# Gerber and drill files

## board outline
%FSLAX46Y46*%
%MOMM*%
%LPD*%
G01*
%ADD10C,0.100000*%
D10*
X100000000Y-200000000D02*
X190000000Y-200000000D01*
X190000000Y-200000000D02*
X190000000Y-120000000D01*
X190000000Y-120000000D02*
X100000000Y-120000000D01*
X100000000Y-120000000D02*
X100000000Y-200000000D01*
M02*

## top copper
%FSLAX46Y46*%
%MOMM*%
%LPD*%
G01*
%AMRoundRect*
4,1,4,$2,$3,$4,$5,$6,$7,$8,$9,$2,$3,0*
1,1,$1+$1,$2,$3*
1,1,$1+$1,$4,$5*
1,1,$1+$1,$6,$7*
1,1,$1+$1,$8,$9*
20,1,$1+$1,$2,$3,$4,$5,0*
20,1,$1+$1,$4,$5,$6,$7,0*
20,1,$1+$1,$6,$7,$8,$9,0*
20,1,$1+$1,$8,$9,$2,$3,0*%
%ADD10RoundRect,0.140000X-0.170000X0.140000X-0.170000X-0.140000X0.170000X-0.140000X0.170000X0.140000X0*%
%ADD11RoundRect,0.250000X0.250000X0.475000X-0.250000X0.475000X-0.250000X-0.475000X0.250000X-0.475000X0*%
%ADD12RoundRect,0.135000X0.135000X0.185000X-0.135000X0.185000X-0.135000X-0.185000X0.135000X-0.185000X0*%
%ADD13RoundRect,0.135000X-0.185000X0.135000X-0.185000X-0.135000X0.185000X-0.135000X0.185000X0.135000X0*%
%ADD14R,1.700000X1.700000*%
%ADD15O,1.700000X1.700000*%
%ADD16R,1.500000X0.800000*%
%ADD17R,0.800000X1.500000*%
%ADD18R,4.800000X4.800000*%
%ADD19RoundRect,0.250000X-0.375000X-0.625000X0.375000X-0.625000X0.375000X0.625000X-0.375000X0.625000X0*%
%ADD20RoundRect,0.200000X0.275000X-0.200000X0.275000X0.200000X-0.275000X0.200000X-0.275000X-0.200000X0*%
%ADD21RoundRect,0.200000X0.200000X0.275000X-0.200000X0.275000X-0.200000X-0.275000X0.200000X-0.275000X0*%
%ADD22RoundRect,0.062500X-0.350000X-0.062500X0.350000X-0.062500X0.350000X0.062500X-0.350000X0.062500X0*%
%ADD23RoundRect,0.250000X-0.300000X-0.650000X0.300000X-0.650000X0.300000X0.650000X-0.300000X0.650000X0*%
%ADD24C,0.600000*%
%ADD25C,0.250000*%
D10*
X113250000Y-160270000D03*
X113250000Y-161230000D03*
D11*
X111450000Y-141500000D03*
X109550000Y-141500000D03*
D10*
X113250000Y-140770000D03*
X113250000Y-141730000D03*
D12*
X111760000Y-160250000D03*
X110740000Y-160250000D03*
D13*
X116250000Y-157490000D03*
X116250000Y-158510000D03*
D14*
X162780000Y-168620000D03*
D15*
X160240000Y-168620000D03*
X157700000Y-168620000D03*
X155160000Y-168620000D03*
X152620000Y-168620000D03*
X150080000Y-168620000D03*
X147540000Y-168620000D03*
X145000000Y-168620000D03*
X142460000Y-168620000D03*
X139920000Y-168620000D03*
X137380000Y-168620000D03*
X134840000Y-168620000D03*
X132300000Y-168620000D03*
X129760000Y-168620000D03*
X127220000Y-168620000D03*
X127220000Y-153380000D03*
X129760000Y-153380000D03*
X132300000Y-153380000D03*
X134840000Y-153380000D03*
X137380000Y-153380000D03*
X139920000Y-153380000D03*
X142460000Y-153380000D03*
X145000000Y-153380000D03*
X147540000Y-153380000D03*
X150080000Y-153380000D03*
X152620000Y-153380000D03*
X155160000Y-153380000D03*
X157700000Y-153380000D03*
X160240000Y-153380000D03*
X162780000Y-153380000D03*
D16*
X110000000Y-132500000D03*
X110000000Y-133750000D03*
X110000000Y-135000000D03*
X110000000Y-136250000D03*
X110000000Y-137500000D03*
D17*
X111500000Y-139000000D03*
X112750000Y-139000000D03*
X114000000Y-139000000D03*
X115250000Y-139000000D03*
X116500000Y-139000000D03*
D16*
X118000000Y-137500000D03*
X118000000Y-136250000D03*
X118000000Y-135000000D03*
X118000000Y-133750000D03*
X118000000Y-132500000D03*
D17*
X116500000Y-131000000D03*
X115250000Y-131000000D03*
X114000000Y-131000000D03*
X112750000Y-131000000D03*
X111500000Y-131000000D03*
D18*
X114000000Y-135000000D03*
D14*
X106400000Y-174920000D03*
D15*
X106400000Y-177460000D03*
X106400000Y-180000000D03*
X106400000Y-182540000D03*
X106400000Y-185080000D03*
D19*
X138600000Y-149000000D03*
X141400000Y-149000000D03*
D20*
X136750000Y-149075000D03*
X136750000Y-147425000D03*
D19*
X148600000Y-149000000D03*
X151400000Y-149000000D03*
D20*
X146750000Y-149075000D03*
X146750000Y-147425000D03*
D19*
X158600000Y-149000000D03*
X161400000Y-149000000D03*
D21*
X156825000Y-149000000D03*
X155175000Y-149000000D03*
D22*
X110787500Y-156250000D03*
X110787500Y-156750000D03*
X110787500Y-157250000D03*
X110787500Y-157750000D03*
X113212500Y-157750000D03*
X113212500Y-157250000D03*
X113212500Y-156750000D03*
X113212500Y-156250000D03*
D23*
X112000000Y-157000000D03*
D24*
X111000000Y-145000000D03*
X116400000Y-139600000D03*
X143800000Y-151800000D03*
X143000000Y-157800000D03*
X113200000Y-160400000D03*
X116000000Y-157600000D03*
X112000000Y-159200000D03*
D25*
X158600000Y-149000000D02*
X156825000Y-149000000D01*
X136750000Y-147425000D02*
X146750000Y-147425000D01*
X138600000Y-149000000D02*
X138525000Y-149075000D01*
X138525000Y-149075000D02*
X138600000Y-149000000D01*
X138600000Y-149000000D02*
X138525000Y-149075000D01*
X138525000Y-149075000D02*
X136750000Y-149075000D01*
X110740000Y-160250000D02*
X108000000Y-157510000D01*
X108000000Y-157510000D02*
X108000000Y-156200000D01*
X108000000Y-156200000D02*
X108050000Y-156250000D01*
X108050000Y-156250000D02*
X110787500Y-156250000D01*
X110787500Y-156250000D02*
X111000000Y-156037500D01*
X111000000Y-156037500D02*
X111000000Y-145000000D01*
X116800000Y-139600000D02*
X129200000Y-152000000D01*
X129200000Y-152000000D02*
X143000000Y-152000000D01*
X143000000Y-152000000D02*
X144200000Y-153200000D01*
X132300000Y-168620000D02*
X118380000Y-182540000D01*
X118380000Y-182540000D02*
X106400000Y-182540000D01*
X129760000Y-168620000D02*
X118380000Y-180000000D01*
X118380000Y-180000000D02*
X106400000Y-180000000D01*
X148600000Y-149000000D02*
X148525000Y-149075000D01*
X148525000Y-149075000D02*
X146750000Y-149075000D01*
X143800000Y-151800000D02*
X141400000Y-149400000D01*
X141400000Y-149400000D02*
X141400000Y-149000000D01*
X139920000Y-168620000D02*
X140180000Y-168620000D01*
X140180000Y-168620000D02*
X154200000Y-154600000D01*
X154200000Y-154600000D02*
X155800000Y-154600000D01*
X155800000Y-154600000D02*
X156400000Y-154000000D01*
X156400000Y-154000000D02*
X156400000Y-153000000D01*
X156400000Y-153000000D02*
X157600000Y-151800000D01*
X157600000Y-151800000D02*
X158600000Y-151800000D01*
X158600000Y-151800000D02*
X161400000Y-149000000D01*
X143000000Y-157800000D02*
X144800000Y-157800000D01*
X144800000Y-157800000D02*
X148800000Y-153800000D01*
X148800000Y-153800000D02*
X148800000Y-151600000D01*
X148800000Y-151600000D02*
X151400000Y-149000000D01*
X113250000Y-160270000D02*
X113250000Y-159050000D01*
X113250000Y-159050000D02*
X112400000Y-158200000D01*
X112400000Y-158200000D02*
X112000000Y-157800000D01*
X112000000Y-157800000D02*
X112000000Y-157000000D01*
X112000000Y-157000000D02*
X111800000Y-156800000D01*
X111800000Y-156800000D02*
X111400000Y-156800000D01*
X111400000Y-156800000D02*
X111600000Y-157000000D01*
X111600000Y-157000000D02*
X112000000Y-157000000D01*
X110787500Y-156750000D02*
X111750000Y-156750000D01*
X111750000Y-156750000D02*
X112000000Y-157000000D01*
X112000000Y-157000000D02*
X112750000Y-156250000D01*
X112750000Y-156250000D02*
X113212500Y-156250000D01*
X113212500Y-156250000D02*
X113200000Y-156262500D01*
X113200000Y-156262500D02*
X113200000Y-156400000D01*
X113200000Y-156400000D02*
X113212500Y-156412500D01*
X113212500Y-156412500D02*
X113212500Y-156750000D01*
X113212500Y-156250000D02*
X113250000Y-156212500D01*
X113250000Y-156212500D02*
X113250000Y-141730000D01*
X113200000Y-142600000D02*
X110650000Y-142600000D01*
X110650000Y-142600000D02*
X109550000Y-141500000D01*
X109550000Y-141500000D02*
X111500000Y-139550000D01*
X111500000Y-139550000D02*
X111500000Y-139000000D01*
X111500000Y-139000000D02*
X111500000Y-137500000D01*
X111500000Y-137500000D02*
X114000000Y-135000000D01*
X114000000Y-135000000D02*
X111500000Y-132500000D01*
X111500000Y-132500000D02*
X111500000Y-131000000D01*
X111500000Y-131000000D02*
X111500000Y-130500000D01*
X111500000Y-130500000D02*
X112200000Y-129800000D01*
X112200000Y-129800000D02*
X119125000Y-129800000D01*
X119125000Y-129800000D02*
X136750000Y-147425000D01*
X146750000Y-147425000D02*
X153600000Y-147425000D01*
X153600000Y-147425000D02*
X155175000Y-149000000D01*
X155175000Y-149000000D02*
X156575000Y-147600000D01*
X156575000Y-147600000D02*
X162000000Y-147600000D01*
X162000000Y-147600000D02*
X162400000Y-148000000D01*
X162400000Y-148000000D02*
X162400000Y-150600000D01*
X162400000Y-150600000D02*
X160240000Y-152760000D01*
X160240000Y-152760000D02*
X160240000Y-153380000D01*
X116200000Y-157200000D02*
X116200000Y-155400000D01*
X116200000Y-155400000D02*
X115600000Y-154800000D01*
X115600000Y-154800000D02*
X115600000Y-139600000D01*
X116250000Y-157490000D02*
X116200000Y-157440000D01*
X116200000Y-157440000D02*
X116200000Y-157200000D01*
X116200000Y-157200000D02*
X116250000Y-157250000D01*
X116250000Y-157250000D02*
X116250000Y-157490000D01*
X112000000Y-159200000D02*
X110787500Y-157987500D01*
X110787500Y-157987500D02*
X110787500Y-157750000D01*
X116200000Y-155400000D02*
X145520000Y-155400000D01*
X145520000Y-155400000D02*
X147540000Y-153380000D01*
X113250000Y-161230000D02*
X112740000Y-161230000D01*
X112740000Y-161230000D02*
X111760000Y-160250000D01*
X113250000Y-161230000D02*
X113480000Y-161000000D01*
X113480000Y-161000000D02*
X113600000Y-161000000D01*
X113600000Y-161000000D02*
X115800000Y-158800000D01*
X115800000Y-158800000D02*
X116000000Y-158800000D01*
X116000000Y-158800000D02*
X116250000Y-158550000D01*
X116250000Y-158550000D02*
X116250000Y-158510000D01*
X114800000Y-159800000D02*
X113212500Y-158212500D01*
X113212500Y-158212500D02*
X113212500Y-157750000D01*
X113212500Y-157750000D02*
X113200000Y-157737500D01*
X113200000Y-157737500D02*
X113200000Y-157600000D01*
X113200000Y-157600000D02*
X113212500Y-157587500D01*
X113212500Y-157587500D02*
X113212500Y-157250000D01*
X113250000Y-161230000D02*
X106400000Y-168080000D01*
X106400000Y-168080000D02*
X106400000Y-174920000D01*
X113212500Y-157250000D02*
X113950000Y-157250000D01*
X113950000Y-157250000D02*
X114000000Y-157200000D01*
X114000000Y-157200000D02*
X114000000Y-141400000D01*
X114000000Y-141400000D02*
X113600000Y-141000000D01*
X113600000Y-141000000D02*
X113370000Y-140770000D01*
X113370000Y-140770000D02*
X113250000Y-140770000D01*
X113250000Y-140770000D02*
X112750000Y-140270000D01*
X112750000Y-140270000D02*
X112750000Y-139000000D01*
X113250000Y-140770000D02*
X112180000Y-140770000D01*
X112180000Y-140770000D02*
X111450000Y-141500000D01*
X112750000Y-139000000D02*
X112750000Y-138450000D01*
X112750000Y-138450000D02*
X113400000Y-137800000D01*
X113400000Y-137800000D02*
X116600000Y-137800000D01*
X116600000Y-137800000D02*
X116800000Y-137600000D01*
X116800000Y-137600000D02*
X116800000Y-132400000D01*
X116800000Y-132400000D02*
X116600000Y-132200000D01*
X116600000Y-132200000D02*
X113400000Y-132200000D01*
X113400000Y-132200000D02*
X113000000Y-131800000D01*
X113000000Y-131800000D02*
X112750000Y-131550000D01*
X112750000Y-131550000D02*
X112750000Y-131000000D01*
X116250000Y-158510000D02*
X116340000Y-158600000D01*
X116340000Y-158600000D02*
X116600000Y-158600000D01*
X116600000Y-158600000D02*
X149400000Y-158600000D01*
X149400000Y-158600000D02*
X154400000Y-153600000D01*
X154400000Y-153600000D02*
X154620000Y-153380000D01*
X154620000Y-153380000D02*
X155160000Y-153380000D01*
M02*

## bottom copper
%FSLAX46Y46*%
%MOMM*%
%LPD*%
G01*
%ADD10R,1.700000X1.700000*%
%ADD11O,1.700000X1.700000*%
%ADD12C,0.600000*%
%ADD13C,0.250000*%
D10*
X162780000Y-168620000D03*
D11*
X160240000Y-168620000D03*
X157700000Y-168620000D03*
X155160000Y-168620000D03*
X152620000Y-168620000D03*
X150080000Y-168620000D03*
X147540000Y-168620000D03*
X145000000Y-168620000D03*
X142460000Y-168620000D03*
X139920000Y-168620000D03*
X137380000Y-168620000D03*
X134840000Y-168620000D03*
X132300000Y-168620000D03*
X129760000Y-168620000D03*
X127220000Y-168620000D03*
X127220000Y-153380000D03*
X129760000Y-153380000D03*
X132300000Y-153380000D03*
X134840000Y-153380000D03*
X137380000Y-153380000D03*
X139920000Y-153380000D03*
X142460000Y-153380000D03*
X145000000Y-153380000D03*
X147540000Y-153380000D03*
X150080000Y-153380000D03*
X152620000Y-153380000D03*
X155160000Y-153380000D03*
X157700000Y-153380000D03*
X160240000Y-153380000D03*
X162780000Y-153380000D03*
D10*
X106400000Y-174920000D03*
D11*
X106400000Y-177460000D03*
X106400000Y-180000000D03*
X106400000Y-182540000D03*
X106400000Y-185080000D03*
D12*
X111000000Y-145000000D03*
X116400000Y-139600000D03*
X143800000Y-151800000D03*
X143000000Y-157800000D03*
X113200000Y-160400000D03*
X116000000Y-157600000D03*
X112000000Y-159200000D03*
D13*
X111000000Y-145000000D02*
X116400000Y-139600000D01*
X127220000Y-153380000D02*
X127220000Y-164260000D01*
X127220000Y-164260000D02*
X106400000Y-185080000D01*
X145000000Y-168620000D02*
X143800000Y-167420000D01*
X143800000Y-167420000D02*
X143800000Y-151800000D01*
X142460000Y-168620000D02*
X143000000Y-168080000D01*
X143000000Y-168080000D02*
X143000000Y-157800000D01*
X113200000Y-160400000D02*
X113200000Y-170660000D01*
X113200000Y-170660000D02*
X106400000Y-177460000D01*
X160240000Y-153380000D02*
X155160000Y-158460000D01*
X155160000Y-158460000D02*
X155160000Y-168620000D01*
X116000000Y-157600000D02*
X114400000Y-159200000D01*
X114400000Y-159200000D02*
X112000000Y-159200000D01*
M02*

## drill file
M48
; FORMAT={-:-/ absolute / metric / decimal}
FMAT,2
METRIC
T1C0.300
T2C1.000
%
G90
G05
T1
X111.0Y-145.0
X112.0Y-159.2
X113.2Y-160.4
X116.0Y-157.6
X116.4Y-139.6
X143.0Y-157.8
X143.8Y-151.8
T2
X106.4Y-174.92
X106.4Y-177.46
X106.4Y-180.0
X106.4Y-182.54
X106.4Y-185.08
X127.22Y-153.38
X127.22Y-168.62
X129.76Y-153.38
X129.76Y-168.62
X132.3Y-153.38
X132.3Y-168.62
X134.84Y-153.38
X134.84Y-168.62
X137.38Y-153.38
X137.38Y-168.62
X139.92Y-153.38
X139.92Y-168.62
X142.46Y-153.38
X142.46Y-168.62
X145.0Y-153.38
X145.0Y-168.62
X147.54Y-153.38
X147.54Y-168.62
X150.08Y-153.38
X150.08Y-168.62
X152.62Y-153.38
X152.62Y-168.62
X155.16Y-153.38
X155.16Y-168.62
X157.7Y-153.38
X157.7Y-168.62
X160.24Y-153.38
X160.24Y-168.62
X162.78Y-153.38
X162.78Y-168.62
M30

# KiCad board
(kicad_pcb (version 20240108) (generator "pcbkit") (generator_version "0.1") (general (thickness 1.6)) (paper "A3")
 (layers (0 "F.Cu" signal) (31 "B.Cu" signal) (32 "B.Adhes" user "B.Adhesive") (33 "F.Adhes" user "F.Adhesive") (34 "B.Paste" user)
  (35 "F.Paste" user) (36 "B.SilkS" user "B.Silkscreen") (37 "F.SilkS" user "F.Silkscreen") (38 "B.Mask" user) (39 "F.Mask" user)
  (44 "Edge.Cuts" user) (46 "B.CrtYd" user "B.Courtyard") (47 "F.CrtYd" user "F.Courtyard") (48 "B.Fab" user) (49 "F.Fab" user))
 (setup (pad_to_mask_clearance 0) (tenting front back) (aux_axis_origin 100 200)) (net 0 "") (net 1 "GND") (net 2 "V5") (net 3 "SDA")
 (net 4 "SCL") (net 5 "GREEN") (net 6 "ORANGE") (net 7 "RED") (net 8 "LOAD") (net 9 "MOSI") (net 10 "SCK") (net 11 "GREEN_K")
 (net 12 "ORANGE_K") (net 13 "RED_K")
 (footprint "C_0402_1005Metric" (layer "F.Cu") (at 113.25 160.75 270)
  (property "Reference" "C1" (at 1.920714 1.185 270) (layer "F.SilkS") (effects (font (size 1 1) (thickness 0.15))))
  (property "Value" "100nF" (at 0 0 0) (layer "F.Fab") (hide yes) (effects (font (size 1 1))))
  (pad "1" smd roundrect (at -0.48 0 270) (size 0.56 0.62) (layers "F.Cu" "F.Paste" "F.Mask") (roundrect_rratio 0.250000000000)
   (solder_mask_margin 0.05) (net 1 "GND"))
  (pad "2" smd roundrect (at 0.48 0 270) (size 0.56 0.62) (layers "F.Cu" "F.Paste" "F.Mask") (roundrect_rratio 0.250000000000)
   (solder_mask_margin 0.05) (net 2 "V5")))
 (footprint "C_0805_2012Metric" (layer "F.Cu") (at 110.5 141.5 180)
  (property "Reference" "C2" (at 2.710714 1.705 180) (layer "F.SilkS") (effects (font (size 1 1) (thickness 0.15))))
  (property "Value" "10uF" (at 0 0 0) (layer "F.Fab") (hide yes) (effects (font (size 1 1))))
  (pad "1" smd roundrect (at -0.95 0 180) (size 1 1.45) (layers "F.Cu" "F.Paste" "F.Mask") (roundrect_rratio 0.250000000000)
   (solder_mask_margin 0.05) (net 2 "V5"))
  (pad "2" smd roundrect (at 0.95 0 180) (size 1 1.45) (layers "F.Cu" "F.Paste" "F.Mask") (roundrect_rratio 0.250000000000)
   (solder_mask_margin 0.05) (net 1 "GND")))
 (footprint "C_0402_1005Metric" (layer "F.Cu") (at 113.25 141.25 270)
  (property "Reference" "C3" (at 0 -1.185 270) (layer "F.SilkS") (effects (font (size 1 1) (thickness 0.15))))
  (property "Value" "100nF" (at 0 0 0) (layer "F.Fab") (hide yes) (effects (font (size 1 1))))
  (pad "1" smd roundrect (at -0.48 0 270) (size 0.56 0.62) (layers "F.Cu" "F.Paste" "F.Mask") (roundrect_rratio 0.250000000000)
   (solder_mask_margin 0.05) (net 2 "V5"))
  (pad "2" smd roundrect (at 0.48 0 270) (size 0.56 0.62) (layers "F.Cu" "F.Paste" "F.Mask") (roundrect_rratio 0.250000000000)
   (solder_mask_margin 0.05) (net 1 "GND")))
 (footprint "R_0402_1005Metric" (layer "F.Cu") (at 111.25 160.25 180)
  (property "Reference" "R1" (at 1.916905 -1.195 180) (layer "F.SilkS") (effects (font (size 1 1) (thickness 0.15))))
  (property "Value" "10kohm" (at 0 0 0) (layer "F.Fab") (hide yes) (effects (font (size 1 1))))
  (pad "1" smd roundrect (at -0.51 0 180) (size 0.54 0.64) (layers "F.Cu" "F.Paste" "F.Mask") (roundrect_rratio 0.250000000000)
   (solder_mask_margin 0.05) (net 2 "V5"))
  (pad "2" smd roundrect (at 0.51 0 180) (size 0.54 0.64) (layers "F.Cu" "F.Paste" "F.Mask") (roundrect_rratio 0.250000000000)
   (solder_mask_margin 0.05) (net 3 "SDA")))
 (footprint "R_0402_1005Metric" (layer "F.Cu") (at 116.25 158 270)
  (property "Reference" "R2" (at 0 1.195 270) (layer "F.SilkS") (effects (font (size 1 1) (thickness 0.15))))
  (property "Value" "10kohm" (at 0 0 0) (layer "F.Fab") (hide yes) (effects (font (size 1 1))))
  (pad "1" smd roundrect (at -0.51 0 270) (size 0.54 0.64) (layers "F.Cu" "F.Paste" "F.Mask") (roundrect_rratio 0.250000000000)
   (solder_mask_margin 0.05) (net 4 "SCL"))
  (pad "2" smd roundrect (at 0.51 0 270) (size 0.54 0.64) (layers "F.Cu" "F.Paste" "F.Mask") (roundrect_rratio 0.250000000000)
   (solder_mask_margin 0.05) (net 2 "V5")))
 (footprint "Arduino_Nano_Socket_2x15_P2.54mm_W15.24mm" (layer "B.Cu") (at 145 161 90)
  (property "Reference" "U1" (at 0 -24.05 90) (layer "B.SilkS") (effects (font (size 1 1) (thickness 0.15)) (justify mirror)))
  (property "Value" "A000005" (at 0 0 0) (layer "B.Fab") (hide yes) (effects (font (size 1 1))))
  (pad "1" thru_hole rect (at -7.62 17.78 90) (size 1.7 1.7) (drill 1) (layers "*.Cu" "*.Mask") (solder_mask_margin 0.05))
  (pad "2" thru_hole oval (at -7.62 15.24 90) (size 1.7 1.7) (drill 1) (layers "*.Cu" "*.Mask") (solder_mask_margin 0.05))
  (pad "3" thru_hole oval (at -7.62 12.7 90) (size 1.7 1.7) (drill 1) (layers "*.Cu" "*.Mask") (solder_mask_margin 0.05))
  (pad "4" thru_hole oval (at -7.62 10.16 90) (size 1.7 1.7) (drill 1) (layers "*.Cu" "*.Mask") (solder_mask_margin 0.05) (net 1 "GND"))
  (pad "5" thru_hole oval (at -7.62 7.62 90) (size 1.7 1.7) (drill 1) (layers "*.Cu" "*.Mask") (solder_mask_margin 0.05))
  (pad "6" thru_hole oval (at -7.62 5.08 90) (size 1.7 1.7) (drill 1) (layers "*.Cu" "*.Mask") (solder_mask_margin 0.05))
  (pad "7" thru_hole oval (at -7.62 2.54 90) (size 1.7 1.7) (drill 1) (layers "*.Cu" "*.Mask") (solder_mask_margin 0.05))
  (pad "8" thru_hole oval (at -7.62 0 90) (size 1.7 1.7) (drill 1) (layers "*.Cu" "*.Mask") (solder_mask_margin 0.05) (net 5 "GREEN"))
  (pad "9" thru_hole oval (at -7.62 -2.54 90) (size 1.7 1.7) (drill 1) (layers "*.Cu" "*.Mask") (solder_mask_margin 0.05) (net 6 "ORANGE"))
  (pad "10" thru_hole oval (at -7.62 -5.08 90) (size 1.7 1.7) (drill 1) (layers "*.Cu" "*.Mask") (solder_mask_margin 0.05) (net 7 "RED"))
  (pad "11" thru_hole oval (at -7.62 -7.62 90) (size 1.7 1.7) (drill 1) (layers "*.Cu" "*.Mask") (solder_mask_margin 0.05))
  (pad "12" thru_hole oval (at -7.62 -10.16 90) (size 1.7 1.7) (drill 1) (layers "*.Cu" "*.Mask") (solder_mask_margin 0.05))
  (pad "13" thru_hole oval (at -7.62 -12.7 90) (size 1.7 1.7) (drill 1) (layers "*.Cu" "*.Mask") (solder_mask_margin 0.05) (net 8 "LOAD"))
  (pad "14" thru_hole oval (at -7.62 -15.24 90) (size 1.7 1.7) (drill 1) (layers "*.Cu" "*.Mask") (solder_mask_margin 0.05) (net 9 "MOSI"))
  (pad "15" thru_hole oval (at -7.62 -17.78 90) (size 1.7 1.7) (drill 1) (layers "*.Cu" "*.Mask") (solder_mask_margin 0.05))
  (pad "16" thru_hole oval (at 7.62 -17.78 90) (size 1.7 1.7) (drill 1) (layers "*.Cu" "*.Mask") (solder_mask_margin 0.05) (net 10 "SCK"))
  (pad "17" thru_hole oval (at 7.62 -15.24 90) (size 1.7 1.7) (drill 1) (layers "*.Cu" "*.Mask") (solder_mask_margin 0.05))
  (pad "18" thru_hole oval (at 7.62 -12.7 90) (size 1.7 1.7) (drill 1) (layers "*.Cu" "*.Mask") (solder_mask_margin 0.05))
  (pad "19" thru_hole oval (at 7.62 -10.16 90) (size 1.7 1.7) (drill 1) (layers "*.Cu" "*.Mask") (solder_mask_margin 0.05))
  (pad "20" thru_hole oval (at 7.62 -7.62 90) (size 1.7 1.7) (drill 1) (layers "*.Cu" "*.Mask") (solder_mask_margin 0.05))
  (pad "21" thru_hole oval (at 7.62 -5.08 90) (size 1.7 1.7) (drill 1) (layers "*.Cu" "*.Mask") (solder_mask_margin 0.05))
  (pad "22" thru_hole oval (at 7.62 -2.54 90) (size 1.7 1.7) (drill 1) (layers "*.Cu" "*.Mask") (solder_mask_margin 0.05))
  (pad "23" thru_hole oval (at 7.62 0 90) (size 1.7 1.7) (drill 1) (layers "*.Cu" "*.Mask") (solder_mask_margin 0.05) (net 3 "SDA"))
  (pad "24" thru_hole oval (at 7.62 2.54 90) (size 1.7 1.7) (drill 1) (layers "*.Cu" "*.Mask") (solder_mask_margin 0.05) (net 4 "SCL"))
  (pad "25" thru_hole oval (at 7.62 5.08 90) (size 1.7 1.7) (drill 1) (layers "*.Cu" "*.Mask") (solder_mask_margin 0.05))
  (pad "26" thru_hole oval (at 7.62 7.62 90) (size 1.7 1.7) (drill 1) (layers "*.Cu" "*.Mask") (solder_mask_margin 0.05))
  (pad "27" thru_hole oval (at 7.62 10.16 90) (size 1.7 1.7) (drill 1) (layers "*.Cu" "*.Mask") (solder_mask_margin 0.05) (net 2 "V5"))
  (pad "28" thru_hole oval (at 7.62 12.7 90) (size 1.7 1.7) (drill 1) (layers "*.Cu" "*.Mask") (solder_mask_margin 0.05))
  (pad "29" thru_hole oval (at 7.62 15.24 90) (size 1.7 1.7) (drill 1) (layers "*.Cu" "*.Mask") (solder_mask_margin 0.05) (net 1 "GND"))
  (pad "30" thru_hole oval (at 7.62 17.78 90) (size 1.7 1.7) (drill 1) (layers "*.Cu" "*.Mask") (solder_mask_margin 0.05)))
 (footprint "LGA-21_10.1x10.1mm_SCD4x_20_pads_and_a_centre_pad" (layer "F.Cu") (at 114 135 0)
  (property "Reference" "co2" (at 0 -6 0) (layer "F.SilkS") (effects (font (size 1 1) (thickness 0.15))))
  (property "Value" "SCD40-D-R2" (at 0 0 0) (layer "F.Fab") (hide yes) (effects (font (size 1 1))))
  (pad "1" smd rect (at -4 -2.5 0) (size 1.5 0.8) (layers "F.Cu" "F.Paste" "F.Mask") (solder_mask_margin 0.05))
  (pad "2" smd rect (at -4 -1.25 0) (size 1.5 0.8) (layers "F.Cu" "F.Paste" "F.Mask") (solder_mask_margin 0.05))
  (pad "3" smd rect (at -4 0 0) (size 1.5 0.8) (layers "F.Cu" "F.Paste" "F.Mask") (solder_mask_margin 0.05))
  (pad "4" smd rect (at -4 1.25 0) (size 1.5 0.8) (layers "F.Cu" "F.Paste" "F.Mask") (solder_mask_margin 0.05))
  (pad "5" smd rect (at -4 2.5 0) (size 1.5 0.8) (layers "F.Cu" "F.Paste" "F.Mask") (solder_mask_margin 0.05))
  (pad "6" smd rect (at -2.5 4 0) (size 0.8 1.5) (layers "F.Cu" "F.Paste" "F.Mask") (solder_mask_margin 0.05) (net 1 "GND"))
  (pad "7" smd rect (at -1.25 4 0) (size 0.8 1.5) (layers "F.Cu" "F.Paste" "F.Mask") (solder_mask_margin 0.05) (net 2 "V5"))
  (pad "8" smd rect (at 0 4 0) (size 0.8 1.5) (layers "F.Cu" "F.Paste" "F.Mask") (solder_mask_margin 0.05))
  (pad "9" smd rect (at 1.25 4 0) (size 0.8 1.5) (layers "F.Cu" "F.Paste" "F.Mask") (solder_mask_margin 0.05) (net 4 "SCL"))
  (pad "10" smd rect (at 2.5 4 0) (size 0.8 1.5) (layers "F.Cu" "F.Paste" "F.Mask") (solder_mask_margin 0.05) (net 3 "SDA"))
  (pad "11" smd rect (at 4 2.5 0) (size 1.5 0.8) (layers "F.Cu" "F.Paste" "F.Mask") (solder_mask_margin 0.05))
  (pad "12" smd rect (at 4 1.25 0) (size 1.5 0.8) (layers "F.Cu" "F.Paste" "F.Mask") (solder_mask_margin 0.05))
  (pad "13" smd rect (at 4 0 0) (size 1.5 0.8) (layers "F.Cu" "F.Paste" "F.Mask") (solder_mask_margin 0.05))
  (pad "14" smd rect (at 4 -1.25 0) (size 1.5 0.8) (layers "F.Cu" "F.Paste" "F.Mask") (solder_mask_margin 0.05))
  (pad "15" smd rect (at 4 -2.5 0) (size 1.5 0.8) (layers "F.Cu" "F.Paste" "F.Mask") (solder_mask_margin 0.05))
  (pad "16" smd rect (at 2.5 -4 0) (size 0.8 1.5) (layers "F.Cu" "F.Paste" "F.Mask") (solder_mask_margin 0.05))
  (pad "17" smd rect (at 1.25 -4 0) (size 0.8 1.5) (layers "F.Cu" "F.Paste" "F.Mask") (solder_mask_margin 0.05))
  (pad "18" smd rect (at 0 -4 0) (size 0.8 1.5) (layers "F.Cu" "F.Paste" "F.Mask") (solder_mask_margin 0.05))
  (pad "19" smd rect (at -1.25 -4 0) (size 0.8 1.5) (layers "F.Cu" "F.Paste" "F.Mask") (solder_mask_margin 0.05) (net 2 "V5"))
  (pad "20" smd rect (at -2.5 -4 0) (size 0.8 1.5) (layers "F.Cu" "F.Paste" "F.Mask") (solder_mask_margin 0.05) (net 1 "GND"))
  (pad "21" smd rect (at 0 0 0) (size 4.8 4.8) (layers "F.Cu" "F.Paste" "F.Mask") (solder_mask_margin 0.05) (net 1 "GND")))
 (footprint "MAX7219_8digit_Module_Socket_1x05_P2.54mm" (layer "F.Cu") (at 145 180 0)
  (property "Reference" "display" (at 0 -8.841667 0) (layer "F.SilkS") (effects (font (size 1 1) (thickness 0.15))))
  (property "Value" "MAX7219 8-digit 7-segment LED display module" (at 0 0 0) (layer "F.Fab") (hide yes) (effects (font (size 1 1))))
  (pad "1" thru_hole rect (at -38.6 -5.08 0) (size 1.7 1.7) (drill 1) (layers "*.Cu" "*.Mask") (solder_mask_margin 0.05) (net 2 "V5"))
  (pad "2" thru_hole oval (at -38.6 -2.54 0) (size 1.7 1.7) (drill 1) (layers "*.Cu" "*.Mask") (solder_mask_margin 0.05) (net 1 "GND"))
  (pad "3" thru_hole oval (at -38.6 0 0) (size 1.7 1.7) (drill 1) (layers "*.Cu" "*.Mask") (solder_mask_margin 0.05) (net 9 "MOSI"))
  (pad "4" thru_hole oval (at -38.6 2.54 0) (size 1.7 1.7) (drill 1) (layers "*.Cu" "*.Mask") (solder_mask_margin 0.05) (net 8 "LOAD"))
  (pad "5" thru_hole oval (at -38.6 5.08 0) (size 1.7 1.7) (drill 1) (layers "*.Cu" "*.Mask") (solder_mask_margin 0.05) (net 10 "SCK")))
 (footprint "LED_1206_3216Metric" (layer "F.Cu") (at 140 149 0)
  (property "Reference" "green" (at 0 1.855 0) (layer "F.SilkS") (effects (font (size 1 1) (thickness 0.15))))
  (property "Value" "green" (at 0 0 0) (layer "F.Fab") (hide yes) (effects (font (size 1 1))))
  (pad "1" smd roundrect (at -1.4 0 0) (size 1.25 1.75) (layers "F.Cu" "F.Paste" "F.Mask") (roundrect_rratio 0.200000000000)
   (solder_mask_margin 0.05) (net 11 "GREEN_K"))
  (pad "2" smd roundrect (at 1.4 0 0) (size 1.25 1.75) (layers "F.Cu" "F.Paste" "F.Mask") (roundrect_rratio 0.200000000000)
   (solder_mask_margin 0.05) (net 5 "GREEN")))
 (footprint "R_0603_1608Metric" (layer "F.Cu") (at 136.75 148.25 90)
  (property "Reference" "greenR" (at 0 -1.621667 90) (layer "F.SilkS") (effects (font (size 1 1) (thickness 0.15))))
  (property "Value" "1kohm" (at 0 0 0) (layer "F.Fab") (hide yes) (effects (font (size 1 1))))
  (pad "1" smd roundrect (at -0.825 0 90) (size 0.8 0.95) (layers "F.Cu" "F.Paste" "F.Mask") (roundrect_rratio 0.250000000000)
   (solder_mask_margin 0.05) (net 11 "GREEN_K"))
  (pad "2" smd roundrect (at 0.825 0 90) (size 0.8 0.95) (layers "F.Cu" "F.Paste" "F.Mask") (roundrect_rratio 0.250000000000)
   (solder_mask_margin 0.05) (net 1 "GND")))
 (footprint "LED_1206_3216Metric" (layer "F.Cu") (at 150 149 0)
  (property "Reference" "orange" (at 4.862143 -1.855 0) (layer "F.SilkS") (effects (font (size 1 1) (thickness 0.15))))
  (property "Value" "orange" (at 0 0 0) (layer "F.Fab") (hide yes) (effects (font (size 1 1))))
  (pad "1" smd roundrect (at -1.4 0 0) (size 1.25 1.75) (layers "F.Cu" "F.Paste" "F.Mask") (roundrect_rratio 0.200000000000)
   (solder_mask_margin 0.05) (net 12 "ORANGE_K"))
  (pad "2" smd roundrect (at 1.4 0 0) (size 1.25 1.75) (layers "F.Cu" "F.Paste" "F.Mask") (roundrect_rratio 0.200000000000)
   (solder_mask_margin 0.05) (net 6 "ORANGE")))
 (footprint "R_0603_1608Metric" (layer "F.Cu") (at 146.75 148.25 90)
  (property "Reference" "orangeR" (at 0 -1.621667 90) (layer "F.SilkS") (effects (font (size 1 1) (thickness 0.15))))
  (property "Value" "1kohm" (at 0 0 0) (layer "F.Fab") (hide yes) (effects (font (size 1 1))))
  (pad "1" smd roundrect (at -0.825 0 90) (size 0.8 0.95) (layers "F.Cu" "F.Paste" "F.Mask") (roundrect_rratio 0.250000000000)
   (solder_mask_margin 0.05) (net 12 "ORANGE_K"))
  (pad "2" smd roundrect (at 0.825 0 90) (size 0.8 0.95) (layers "F.Cu" "F.Paste" "F.Mask") (roundrect_rratio 0.250000000000)
   (solder_mask_margin 0.05) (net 1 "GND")))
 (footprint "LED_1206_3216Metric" (layer "F.Cu") (at 160 149 0)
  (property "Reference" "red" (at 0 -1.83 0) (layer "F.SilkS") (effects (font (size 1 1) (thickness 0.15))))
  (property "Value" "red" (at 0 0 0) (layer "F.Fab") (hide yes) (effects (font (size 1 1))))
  (pad "1" smd roundrect (at -1.4 0 0) (size 1.25 1.75) (layers "F.Cu" "F.Paste" "F.Mask") (roundrect_rratio 0.200000000000)
   (solder_mask_margin 0.05) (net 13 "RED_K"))
  (pad "2" smd roundrect (at 1.4 0 0) (size 1.25 1.75) (layers "F.Cu" "F.Paste" "F.Mask") (roundrect_rratio 0.200000000000)
   (solder_mask_margin 0.05) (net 7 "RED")))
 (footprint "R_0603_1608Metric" (layer "F.Cu") (at 156 149 180)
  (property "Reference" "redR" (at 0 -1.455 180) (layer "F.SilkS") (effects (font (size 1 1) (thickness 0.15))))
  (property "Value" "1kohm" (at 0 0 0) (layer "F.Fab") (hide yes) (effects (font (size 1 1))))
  (pad "1" smd roundrect (at -0.825 0 180) (size 0.8 0.95) (layers "F.Cu" "F.Paste" "F.Mask") (roundrect_rratio 0.250000000000)
   (solder_mask_margin 0.05) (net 13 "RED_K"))
  (pad "2" smd roundrect (at 0.825 0 180) (size 0.8 0.95) (layers "F.Cu" "F.Paste" "F.Mask") (roundrect_rratio 0.250000000000)
   (solder_mask_margin 0.05) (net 1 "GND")))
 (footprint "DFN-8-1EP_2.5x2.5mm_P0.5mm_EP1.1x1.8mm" (layer "F.Cu") (at 112 157 0)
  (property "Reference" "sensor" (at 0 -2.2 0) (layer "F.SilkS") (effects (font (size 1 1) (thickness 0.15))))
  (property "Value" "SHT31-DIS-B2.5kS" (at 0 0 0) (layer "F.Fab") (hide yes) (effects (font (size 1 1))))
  (pad "1" smd roundrect (at -1.2125 -0.75 0) (size 0.825 0.25) (layers "F.Cu" "F.Paste" "F.Mask") (roundrect_rratio 0.250000000000)
   (solder_mask_margin 0.05) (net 3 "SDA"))
  (pad "2" smd roundrect (at -1.2125 -0.25 0) (size 0.825 0.25) (layers "F.Cu" "F.Paste" "F.Mask") (roundrect_rratio 0.250000000000)
   (solder_mask_margin 0.05) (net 1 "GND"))
  (pad "3" smd roundrect (at -1.2125 0.25 0) (size 0.825 0.25) (layers "F.Cu" "F.Paste" "F.Mask") (roundrect_rratio 0.250000000000)
   (solder_mask_margin 0.05))
  (pad "4" smd roundrect (at -1.2125 0.75 0) (size 0.825 0.25) (layers "F.Cu" "F.Paste" "F.Mask") (roundrect_rratio 0.250000000000)
   (solder_mask_margin 0.05) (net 4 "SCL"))
  (pad "5" smd roundrect (at 1.2125 0.75 0) (size 0.825 0.25) (layers "F.Cu" "F.Paste" "F.Mask") (roundrect_rratio 0.250000000000)
   (solder_mask_margin 0.05) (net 2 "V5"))
  (pad "6" smd roundrect (at 1.2125 0.25 0) (size 0.825 0.25) (layers "F.Cu" "F.Paste" "F.Mask") (roundrect_rratio 0.250000000000)
   (solder_mask_margin 0.05) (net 2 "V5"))
  (pad "7" smd roundrect (at 1.2125 -0.25 0) (size 0.825 0.25) (layers "F.Cu" "F.Paste" "F.Mask") (roundrect_rratio 0.250000000000)
   (solder_mask_margin 0.05) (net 1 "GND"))
  (pad "8" smd roundrect (at 1.2125 -0.75 0) (size 0.825 0.25) (layers "F.Cu" "F.Paste" "F.Mask") (roundrect_rratio 0.250000000000)
   (solder_mask_margin 0.05) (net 1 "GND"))
  (pad "9" smd roundrect (at 0 0 0) (size 1.1 1.8) (layers "F.Cu" "F.Paste" "F.Mask") (roundrect_rratio 0.227272727273)
   (solder_mask_margin 0.05) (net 1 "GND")))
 (segment (start 158.6 149) (end 156.825 149) (width 0.25) (layer "F.Cu") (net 13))
 (segment (start 136.75 147.425) (end 146.75 147.425) (width 0.25) (layer "F.Cu") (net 1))
 (segment (start 138.6 149) (end 138.525 149.075) (width 0.25) (layer "F.Cu") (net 11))
 (segment (start 138.525 149.075) (end 138.6 149) (width 0.25) (layer "F.Cu") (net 11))
 (segment (start 138.6 149) (end 138.525 149.075) (width 0.25) (layer "F.Cu") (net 11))
 (segment (start 138.525 149.075) (end 136.75 149.075) (width 0.25) (layer "F.Cu") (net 11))
 (segment (start 110.74 160.25) (end 108 157.51) (width 0.25) (layer "F.Cu") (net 3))
 (segment (start 108 157.51) (end 108 156.2) (width 0.25) (layer "F.Cu") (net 3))
 (segment (start 108 156.2) (end 108.05 156.25) (width 0.25) (layer "F.Cu") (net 3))
 (segment (start 108.05 156.25) (end 110.7875 156.25) (width 0.25) (layer "F.Cu") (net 3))
 (segment (start 110.7875 156.25) (end 111 156.0375) (width 0.25) (layer "F.Cu") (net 3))
 (segment (start 111 156.0375) (end 111 145) (width 0.25) (layer "F.Cu") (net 3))
 (segment (start 111 145) (end 116.4 139.6) (width 0.25) (layer "B.Cu") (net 3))
 (segment (start 116.8 139.6) (end 129.2 152) (width 0.25) (layer "F.Cu") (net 3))
 (segment (start 129.2 152) (end 143 152) (width 0.25) (layer "F.Cu") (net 3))
 (segment (start 143 152) (end 144.2 153.2) (width 0.25) (layer "F.Cu") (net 3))
 (segment (start 127.22 153.38) (end 127.22 164.26) (width 0.25) (layer "B.Cu") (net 10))
 (segment (start 127.22 164.26) (end 106.4 185.08) (width 0.25) (layer "B.Cu") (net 10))
 (segment (start 132.3 168.62) (end 118.38 182.54) (width 0.25) (layer "F.Cu") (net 8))
 (segment (start 118.38 182.54) (end 106.4 182.54) (width 0.25) (layer "F.Cu") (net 8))
 (segment (start 129.76 168.62) (end 118.38 180) (width 0.25) (layer "F.Cu") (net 9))
 (segment (start 118.38 180) (end 106.4 180) (width 0.25) (layer "F.Cu") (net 9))
 (segment (start 148.6 149) (end 148.525 149.075) (width 0.25) (layer "F.Cu") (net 12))
 (segment (start 148.525 149.075) (end 146.75 149.075) (width 0.25) (layer "F.Cu") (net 12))
 (segment (start 145 168.62) (end 143.8 167.42) (width 0.25) (layer "B.Cu") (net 5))
 (segment (start 143.8 167.42) (end 143.8 151.8) (width 0.25) (layer "B.Cu") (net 5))
 (segment (start 143.8 151.8) (end 141.4 149.4) (width 0.25) (layer "F.Cu") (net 5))
 (segment (start 141.4 149.4) (end 141.4 149) (width 0.25) (layer "F.Cu") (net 5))
 (segment (start 139.92 168.62) (end 140.18 168.62) (width 0.25) (layer "F.Cu") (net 7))
 (segment (start 140.18 168.62) (end 154.2 154.6) (width 0.25) (layer "F.Cu") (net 7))
 (segment (start 154.2 154.6) (end 155.8 154.6) (width 0.25) (layer "F.Cu") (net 7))
 (segment (start 155.8 154.6) (end 156.4 154) (width 0.25) (layer "F.Cu") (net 7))
 (segment (start 156.4 154) (end 156.4 153) (width 0.25) (layer "F.Cu") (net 7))
 (segment (start 156.4 153) (end 157.6 151.8) (width 0.25) (layer "F.Cu") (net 7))
 (segment (start 157.6 151.8) (end 158.6 151.8) (width 0.25) (layer "F.Cu") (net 7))
 (segment (start 158.6 151.8) (end 161.4 149) (width 0.25) (layer "F.Cu") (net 7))
 (segment (start 142.46 168.62) (end 143 168.08) (width 0.25) (layer "B.Cu") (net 6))
 (segment (start 143 168.08) (end 143 157.8) (width 0.25) (layer "B.Cu") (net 6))
 (segment (start 143 157.8) (end 144.8 157.8) (width 0.25) (layer "F.Cu") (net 6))
 (segment (start 144.8 157.8) (end 148.8 153.8) (width 0.25) (layer "F.Cu") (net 6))
 (segment (start 148.8 153.8) (end 148.8 151.6) (width 0.25) (layer "F.Cu") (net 6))
 (segment (start 148.8 151.6) (end 151.4 149) (width 0.25) (layer "F.Cu") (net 6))
 (segment (start 113.25 160.27) (end 113.25 159.05) (width 0.25) (layer "F.Cu") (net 1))
 (segment (start 113.25 159.05) (end 112.4 158.2) (width 0.25) (layer "F.Cu") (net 1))
 (segment (start 112.4 158.2) (end 112 157.8) (width 0.25) (layer "F.Cu") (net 1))
 (segment (start 112 157.8) (end 112 157) (width 0.25) (layer "F.Cu") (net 1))
 (segment (start 112 157) (end 111.8 156.8) (width 0.25) (layer "F.Cu") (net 1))
 (segment (start 111.8 156.8) (end 111.4 156.8) (width 0.25) (layer "F.Cu") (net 1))
 (segment (start 111.4 156.8) (end 111.6 157) (width 0.25) (layer "F.Cu") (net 1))
 (segment (start 111.6 157) (end 112 157) (width 0.25) (layer "F.Cu") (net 1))
 (segment (start 110.7875 156.75) (end 111.75 156.75) (width 0.25) (layer "F.Cu") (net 1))
 (segment (start 111.75 156.75) (end 112 157) (width 0.25) (layer "F.Cu") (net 1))
 (segment (start 112 157) (end 112.75 156.25) (width 0.25) (layer "F.Cu") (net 1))
 (segment (start 112.75 156.25) (end 113.2125 156.25) (width 0.25) (layer "F.Cu") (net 1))
 (segment (start 113.2125 156.25) (end 113.2 156.2625) (width 0.25) (layer "F.Cu") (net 1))
 (segment (start 113.2 156.2625) (end 113.2 156.4) (width 0.25) (layer "F.Cu") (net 1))
 (segment (start 113.2 156.4) (end 113.2125 156.4125) (width 0.25) (layer "F.Cu") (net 1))
 (segment (start 113.2125 156.4125) (end 113.2125 156.75) (width 0.25) (layer "F.Cu") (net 1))
 (segment (start 113.2125 156.25) (end 113.25 156.2125) (width 0.25) (layer "F.Cu") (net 1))
 (segment (start 113.25 156.2125) (end 113.25 141.73) (width 0.25) (layer "F.Cu") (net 1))
 (segment (start 113.2 142.6) (end 110.65 142.6) (width 0.25) (layer "F.Cu") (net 1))
 (segment (start 110.65 142.6) (end 109.55 141.5) (width 0.25) (layer "F.Cu") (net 1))
 (segment (start 109.55 141.5) (end 111.5 139.55) (width 0.25) (layer "F.Cu") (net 1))
 (segment (start 111.5 139.55) (end 111.5 139) (width 0.25) (layer "F.Cu") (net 1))
 (segment (start 111.5 139) (end 111.5 137.5) (width 0.25) (layer "F.Cu") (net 1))
 (segment (start 111.5 137.5) (end 114 135) (width 0.25) (layer "F.Cu") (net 1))
 (segment (start 114 135) (end 111.5 132.5) (width 0.25) (layer "F.Cu") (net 1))
 (segment (start 111.5 132.5) (end 111.5 131) (width 0.25) (layer "F.Cu") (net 1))
 (segment (start 113.2 160.4) (end 113.2 170.66) (width 0.25) (layer "B.Cu") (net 1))
 (segment (start 113.2 170.66) (end 106.4 177.46) (width 0.25) (layer "B.Cu") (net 1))
 (segment (start 111.5 131) (end 111.5 130.5) (width 0.25) (layer "F.Cu") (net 1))
 (segment (start 111.5 130.5) (end 112.2 129.8) (width 0.25) (layer "F.Cu") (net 1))
 (segment (start 112.2 129.8) (end 119.125 129.8) (width 0.25) (layer "F.Cu") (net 1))
 (segment (start 119.125 129.8) (end 136.75 147.425) (width 0.25) (layer "F.Cu") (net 1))
 (segment (start 146.75 147.425) (end 153.6 147.425) (width 0.25) (layer "F.Cu") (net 1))
 (segment (start 153.6 147.425) (end 155.175 149) (width 0.25) (layer "F.Cu") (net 1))
 (segment (start 155.175 149) (end 156.575 147.6) (width 0.25) (layer "F.Cu") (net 1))
 (segment (start 156.575 147.6) (end 162 147.6) (width 0.25) (layer "F.Cu") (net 1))
 (segment (start 162 147.6) (end 162.4 148) (width 0.25) (layer "F.Cu") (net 1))
 (segment (start 162.4 148) (end 162.4 150.6) (width 0.25) (layer "F.Cu") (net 1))
 (segment (start 162.4 150.6) (end 160.24 152.76) (width 0.25) (layer "F.Cu") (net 1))
 (segment (start 160.24 152.76) (end 160.24 153.38) (width 0.25) (layer "F.Cu") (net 1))
 (segment (start 160.24 153.38) (end 155.16 158.46) (width 0.25) (layer "B.Cu") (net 1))
 (segment (start 155.16 158.46) (end 155.16 168.62) (width 0.25) (layer "B.Cu") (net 1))
 (segment (start 116.2 157.2) (end 116.2 155.4) (width 0.25) (layer "F.Cu") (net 4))
 (segment (start 116.2 155.4) (end 115.6 154.8) (width 0.25) (layer "F.Cu") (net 4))
 (segment (start 115.6 154.8) (end 115.6 139.6) (width 0.25) (layer "F.Cu") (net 4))
 (segment (start 116.25 157.49) (end 116.2 157.44) (width 0.25) (layer "F.Cu") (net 4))
 (segment (start 116.2 157.44) (end 116.2 157.2) (width 0.25) (layer "F.Cu") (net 4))
 (segment (start 116.2 157.2) (end 116.25 157.25) (width 0.25) (layer "F.Cu") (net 4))
 (segment (start 116.25 157.25) (end 116.25 157.49) (width 0.25) (layer "F.Cu") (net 4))
 (segment (start 116 157.6) (end 114.4 159.2) (width 0.25) (layer "B.Cu") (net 4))
 (segment (start 114.4 159.2) (end 112 159.2) (width 0.25) (layer "B.Cu") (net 4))
 (segment (start 112 159.2) (end 110.7875 157.9875) (width 0.25) (layer "F.Cu") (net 4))
 (segment (start 110.7875 157.9875) (end 110.7875 157.75) (width 0.25) (layer "F.Cu") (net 4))
 (segment (start 116.2 155.4) (end 145.52 155.4) (width 0.25) (layer "F.Cu") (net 4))
 (segment (start 145.52 155.4) (end 147.54 153.38) (width 0.25) (layer "F.Cu") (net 4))
 (segment (start 113.25 161.23) (end 112.74 161.23) (width 0.25) (layer "F.Cu") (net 2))
 (segment (start 112.74 161.23) (end 111.76 160.25) (width 0.25) (layer "F.Cu") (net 2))
 (segment (start 113.25 161.23) (end 113.48 161) (width 0.25) (layer "F.Cu") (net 2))
 (segment (start 113.48 161) (end 113.6 161) (width 0.25) (layer "F.Cu") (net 2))
 (segment (start 113.6 161) (end 115.8 158.8) (width 0.25) (layer "F.Cu") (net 2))
 (segment (start 115.8 158.8) (end 116 158.8) (width 0.25) (layer "F.Cu") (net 2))
 (segment (start 116 158.8) (end 116.25 158.55) (width 0.25) (layer "F.Cu") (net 2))
 (segment (start 116.25 158.55) (end 116.25 158.51) (width 0.25) (layer "F.Cu") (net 2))
 (segment (start 114.8 159.8) (end 113.2125 158.2125) (width 0.25) (layer "F.Cu") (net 2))
 (segment (start 113.2125 158.2125) (end 113.2125 157.75) (width 0.25) (layer "F.Cu") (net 2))
 (segment (start 113.2125 157.75) (end 113.2 157.7375) (width 0.25) (layer "F.Cu") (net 2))
 (segment (start 113.2 157.7375) (end 113.2 157.6) (width 0.25) (layer "F.Cu") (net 2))
 (segment (start 113.2 157.6) (end 113.2125 157.5875) (width 0.25) (layer "F.Cu") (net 2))
 (segment (start 113.2125 157.5875) (end 113.2125 157.25) (width 0.25) (layer "F.Cu") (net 2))
 (segment (start 113.25 161.23) (end 106.4 168.08) (width 0.25) (layer "F.Cu") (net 2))
 (segment (start 106.4 168.08) (end 106.4 174.92) (width 0.25) (layer "F.Cu") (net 2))
 (segment (start 113.2125 157.25) (end 113.95 157.25) (width 0.25) (layer "F.Cu") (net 2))
 (segment (start 113.95 157.25) (end 114 157.2) (width 0.25) (layer "F.Cu") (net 2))
 (segment (start 114 157.2) (end 114 141.4) (width 0.25) (layer "F.Cu") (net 2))
 (segment (start 114 141.4) (end 113.6 141) (width 0.25) (layer "F.Cu") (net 2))
 (segment (start 113.6 141) (end 113.37 140.77) (width 0.25) (layer "F.Cu") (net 2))
 (segment (start 113.37 140.77) (end 113.25 140.77) (width 0.25) (layer "F.Cu") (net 2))
 (segment (start 113.25 140.77) (end 112.75 140.27) (width 0.25) (layer "F.Cu") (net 2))
 (segment (start 112.75 140.27) (end 112.75 139) (width 0.25) (layer "F.Cu") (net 2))
 (segment (start 113.25 140.77) (end 112.18 140.77) (width 0.25) (layer "F.Cu") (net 2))
 (segment (start 112.18 140.77) (end 111.45 141.5) (width 0.25) (layer "F.Cu") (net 2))
 (segment (start 112.75 139) (end 112.75 138.45) (width 0.25) (layer "F.Cu") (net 2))
 (segment (start 112.75 138.45) (end 113.4 137.8) (width 0.25) (layer "F.Cu") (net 2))
 (segment (start 113.4 137.8) (end 116.6 137.8) (width 0.25) (layer "F.Cu") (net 2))
 (segment (start 116.6 137.8) (end 116.8 137.6) (width 0.25) (layer "F.Cu") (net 2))
 (segment (start 116.8 137.6) (end 116.8 132.4) (width 0.25) (layer "F.Cu") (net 2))
 (segment (start 116.8 132.4) (end 116.6 132.2) (width 0.25) (layer "F.Cu") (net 2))
 (segment (start 116.6 132.2) (end 113.4 132.2) (width 0.25) (layer "F.Cu") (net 2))
 (segment (start 113.4 132.2) (end 113 131.8) (width 0.25) (layer "F.Cu") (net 2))
 (segment (start 113 131.8) (end 112.75 131.55) (width 0.25) (layer "F.Cu") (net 2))
 (segment (start 112.75 131.55) (end 112.75 131) (width 0.25) (layer "F.Cu") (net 2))
 (segment (start 116.25 158.51) (end 116.34 158.6) (width 0.25) (layer "F.Cu") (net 2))
 (segment (start 116.34 158.6) (end 116.6 158.6) (width 0.25) (layer "F.Cu") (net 2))
 (segment (start 116.6 158.6) (end 149.4 158.6) (width 0.25) (layer "F.Cu") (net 2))
 (segment (start 149.4 158.6) (end 154.4 153.6) (width 0.25) (layer "F.Cu") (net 2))
 (segment (start 154.4 153.6) (end 154.62 153.38) (width 0.25) (layer "F.Cu") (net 2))
 (segment (start 154.62 153.38) (end 155.16 153.38) (width 0.25) (layer "F.Cu") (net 2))
 (via (at 111 145) (size 0.6) (drill 0.3) (layers "F.Cu" "B.Cu") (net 3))
 (via (at 116.4 139.6) (size 0.6) (drill 0.3) (layers "F.Cu" "B.Cu") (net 3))
 (via (at 143.8 151.8) (size 0.6) (drill 0.3) (layers "F.Cu" "B.Cu") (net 5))
 (via (at 143 157.8) (size 0.6) (drill 0.3) (layers "F.Cu" "B.Cu") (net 6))
 (via (at 113.2 160.4) (size 0.6) (drill 0.3) (layers "F.Cu" "B.Cu") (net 1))
 (via (at 116 157.6) (size 0.6) (drill 0.3) (layers "F.Cu" "B.Cu") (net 4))
 (via (at 112 159.2) (size 0.6) (drill 0.3) (layers "F.Cu" "B.Cu") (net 4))
 (gr_line (start 100 200) (end 190 200) (stroke (width 0.1) (type solid)) (layer "Edge.Cuts"))
 (gr_line (start 190 200) (end 190 120) (stroke (width 0.1) (type solid)) (layer "Edge.Cuts"))
 (gr_line (start 190 120) (end 100 120) (stroke (width 0.1) (type solid)) (layer "Edge.Cuts"))
 (gr_line (start 100 120) (end 100 200) (stroke (width 0.1) (type solid)) (layer "Edge.Cuts")))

